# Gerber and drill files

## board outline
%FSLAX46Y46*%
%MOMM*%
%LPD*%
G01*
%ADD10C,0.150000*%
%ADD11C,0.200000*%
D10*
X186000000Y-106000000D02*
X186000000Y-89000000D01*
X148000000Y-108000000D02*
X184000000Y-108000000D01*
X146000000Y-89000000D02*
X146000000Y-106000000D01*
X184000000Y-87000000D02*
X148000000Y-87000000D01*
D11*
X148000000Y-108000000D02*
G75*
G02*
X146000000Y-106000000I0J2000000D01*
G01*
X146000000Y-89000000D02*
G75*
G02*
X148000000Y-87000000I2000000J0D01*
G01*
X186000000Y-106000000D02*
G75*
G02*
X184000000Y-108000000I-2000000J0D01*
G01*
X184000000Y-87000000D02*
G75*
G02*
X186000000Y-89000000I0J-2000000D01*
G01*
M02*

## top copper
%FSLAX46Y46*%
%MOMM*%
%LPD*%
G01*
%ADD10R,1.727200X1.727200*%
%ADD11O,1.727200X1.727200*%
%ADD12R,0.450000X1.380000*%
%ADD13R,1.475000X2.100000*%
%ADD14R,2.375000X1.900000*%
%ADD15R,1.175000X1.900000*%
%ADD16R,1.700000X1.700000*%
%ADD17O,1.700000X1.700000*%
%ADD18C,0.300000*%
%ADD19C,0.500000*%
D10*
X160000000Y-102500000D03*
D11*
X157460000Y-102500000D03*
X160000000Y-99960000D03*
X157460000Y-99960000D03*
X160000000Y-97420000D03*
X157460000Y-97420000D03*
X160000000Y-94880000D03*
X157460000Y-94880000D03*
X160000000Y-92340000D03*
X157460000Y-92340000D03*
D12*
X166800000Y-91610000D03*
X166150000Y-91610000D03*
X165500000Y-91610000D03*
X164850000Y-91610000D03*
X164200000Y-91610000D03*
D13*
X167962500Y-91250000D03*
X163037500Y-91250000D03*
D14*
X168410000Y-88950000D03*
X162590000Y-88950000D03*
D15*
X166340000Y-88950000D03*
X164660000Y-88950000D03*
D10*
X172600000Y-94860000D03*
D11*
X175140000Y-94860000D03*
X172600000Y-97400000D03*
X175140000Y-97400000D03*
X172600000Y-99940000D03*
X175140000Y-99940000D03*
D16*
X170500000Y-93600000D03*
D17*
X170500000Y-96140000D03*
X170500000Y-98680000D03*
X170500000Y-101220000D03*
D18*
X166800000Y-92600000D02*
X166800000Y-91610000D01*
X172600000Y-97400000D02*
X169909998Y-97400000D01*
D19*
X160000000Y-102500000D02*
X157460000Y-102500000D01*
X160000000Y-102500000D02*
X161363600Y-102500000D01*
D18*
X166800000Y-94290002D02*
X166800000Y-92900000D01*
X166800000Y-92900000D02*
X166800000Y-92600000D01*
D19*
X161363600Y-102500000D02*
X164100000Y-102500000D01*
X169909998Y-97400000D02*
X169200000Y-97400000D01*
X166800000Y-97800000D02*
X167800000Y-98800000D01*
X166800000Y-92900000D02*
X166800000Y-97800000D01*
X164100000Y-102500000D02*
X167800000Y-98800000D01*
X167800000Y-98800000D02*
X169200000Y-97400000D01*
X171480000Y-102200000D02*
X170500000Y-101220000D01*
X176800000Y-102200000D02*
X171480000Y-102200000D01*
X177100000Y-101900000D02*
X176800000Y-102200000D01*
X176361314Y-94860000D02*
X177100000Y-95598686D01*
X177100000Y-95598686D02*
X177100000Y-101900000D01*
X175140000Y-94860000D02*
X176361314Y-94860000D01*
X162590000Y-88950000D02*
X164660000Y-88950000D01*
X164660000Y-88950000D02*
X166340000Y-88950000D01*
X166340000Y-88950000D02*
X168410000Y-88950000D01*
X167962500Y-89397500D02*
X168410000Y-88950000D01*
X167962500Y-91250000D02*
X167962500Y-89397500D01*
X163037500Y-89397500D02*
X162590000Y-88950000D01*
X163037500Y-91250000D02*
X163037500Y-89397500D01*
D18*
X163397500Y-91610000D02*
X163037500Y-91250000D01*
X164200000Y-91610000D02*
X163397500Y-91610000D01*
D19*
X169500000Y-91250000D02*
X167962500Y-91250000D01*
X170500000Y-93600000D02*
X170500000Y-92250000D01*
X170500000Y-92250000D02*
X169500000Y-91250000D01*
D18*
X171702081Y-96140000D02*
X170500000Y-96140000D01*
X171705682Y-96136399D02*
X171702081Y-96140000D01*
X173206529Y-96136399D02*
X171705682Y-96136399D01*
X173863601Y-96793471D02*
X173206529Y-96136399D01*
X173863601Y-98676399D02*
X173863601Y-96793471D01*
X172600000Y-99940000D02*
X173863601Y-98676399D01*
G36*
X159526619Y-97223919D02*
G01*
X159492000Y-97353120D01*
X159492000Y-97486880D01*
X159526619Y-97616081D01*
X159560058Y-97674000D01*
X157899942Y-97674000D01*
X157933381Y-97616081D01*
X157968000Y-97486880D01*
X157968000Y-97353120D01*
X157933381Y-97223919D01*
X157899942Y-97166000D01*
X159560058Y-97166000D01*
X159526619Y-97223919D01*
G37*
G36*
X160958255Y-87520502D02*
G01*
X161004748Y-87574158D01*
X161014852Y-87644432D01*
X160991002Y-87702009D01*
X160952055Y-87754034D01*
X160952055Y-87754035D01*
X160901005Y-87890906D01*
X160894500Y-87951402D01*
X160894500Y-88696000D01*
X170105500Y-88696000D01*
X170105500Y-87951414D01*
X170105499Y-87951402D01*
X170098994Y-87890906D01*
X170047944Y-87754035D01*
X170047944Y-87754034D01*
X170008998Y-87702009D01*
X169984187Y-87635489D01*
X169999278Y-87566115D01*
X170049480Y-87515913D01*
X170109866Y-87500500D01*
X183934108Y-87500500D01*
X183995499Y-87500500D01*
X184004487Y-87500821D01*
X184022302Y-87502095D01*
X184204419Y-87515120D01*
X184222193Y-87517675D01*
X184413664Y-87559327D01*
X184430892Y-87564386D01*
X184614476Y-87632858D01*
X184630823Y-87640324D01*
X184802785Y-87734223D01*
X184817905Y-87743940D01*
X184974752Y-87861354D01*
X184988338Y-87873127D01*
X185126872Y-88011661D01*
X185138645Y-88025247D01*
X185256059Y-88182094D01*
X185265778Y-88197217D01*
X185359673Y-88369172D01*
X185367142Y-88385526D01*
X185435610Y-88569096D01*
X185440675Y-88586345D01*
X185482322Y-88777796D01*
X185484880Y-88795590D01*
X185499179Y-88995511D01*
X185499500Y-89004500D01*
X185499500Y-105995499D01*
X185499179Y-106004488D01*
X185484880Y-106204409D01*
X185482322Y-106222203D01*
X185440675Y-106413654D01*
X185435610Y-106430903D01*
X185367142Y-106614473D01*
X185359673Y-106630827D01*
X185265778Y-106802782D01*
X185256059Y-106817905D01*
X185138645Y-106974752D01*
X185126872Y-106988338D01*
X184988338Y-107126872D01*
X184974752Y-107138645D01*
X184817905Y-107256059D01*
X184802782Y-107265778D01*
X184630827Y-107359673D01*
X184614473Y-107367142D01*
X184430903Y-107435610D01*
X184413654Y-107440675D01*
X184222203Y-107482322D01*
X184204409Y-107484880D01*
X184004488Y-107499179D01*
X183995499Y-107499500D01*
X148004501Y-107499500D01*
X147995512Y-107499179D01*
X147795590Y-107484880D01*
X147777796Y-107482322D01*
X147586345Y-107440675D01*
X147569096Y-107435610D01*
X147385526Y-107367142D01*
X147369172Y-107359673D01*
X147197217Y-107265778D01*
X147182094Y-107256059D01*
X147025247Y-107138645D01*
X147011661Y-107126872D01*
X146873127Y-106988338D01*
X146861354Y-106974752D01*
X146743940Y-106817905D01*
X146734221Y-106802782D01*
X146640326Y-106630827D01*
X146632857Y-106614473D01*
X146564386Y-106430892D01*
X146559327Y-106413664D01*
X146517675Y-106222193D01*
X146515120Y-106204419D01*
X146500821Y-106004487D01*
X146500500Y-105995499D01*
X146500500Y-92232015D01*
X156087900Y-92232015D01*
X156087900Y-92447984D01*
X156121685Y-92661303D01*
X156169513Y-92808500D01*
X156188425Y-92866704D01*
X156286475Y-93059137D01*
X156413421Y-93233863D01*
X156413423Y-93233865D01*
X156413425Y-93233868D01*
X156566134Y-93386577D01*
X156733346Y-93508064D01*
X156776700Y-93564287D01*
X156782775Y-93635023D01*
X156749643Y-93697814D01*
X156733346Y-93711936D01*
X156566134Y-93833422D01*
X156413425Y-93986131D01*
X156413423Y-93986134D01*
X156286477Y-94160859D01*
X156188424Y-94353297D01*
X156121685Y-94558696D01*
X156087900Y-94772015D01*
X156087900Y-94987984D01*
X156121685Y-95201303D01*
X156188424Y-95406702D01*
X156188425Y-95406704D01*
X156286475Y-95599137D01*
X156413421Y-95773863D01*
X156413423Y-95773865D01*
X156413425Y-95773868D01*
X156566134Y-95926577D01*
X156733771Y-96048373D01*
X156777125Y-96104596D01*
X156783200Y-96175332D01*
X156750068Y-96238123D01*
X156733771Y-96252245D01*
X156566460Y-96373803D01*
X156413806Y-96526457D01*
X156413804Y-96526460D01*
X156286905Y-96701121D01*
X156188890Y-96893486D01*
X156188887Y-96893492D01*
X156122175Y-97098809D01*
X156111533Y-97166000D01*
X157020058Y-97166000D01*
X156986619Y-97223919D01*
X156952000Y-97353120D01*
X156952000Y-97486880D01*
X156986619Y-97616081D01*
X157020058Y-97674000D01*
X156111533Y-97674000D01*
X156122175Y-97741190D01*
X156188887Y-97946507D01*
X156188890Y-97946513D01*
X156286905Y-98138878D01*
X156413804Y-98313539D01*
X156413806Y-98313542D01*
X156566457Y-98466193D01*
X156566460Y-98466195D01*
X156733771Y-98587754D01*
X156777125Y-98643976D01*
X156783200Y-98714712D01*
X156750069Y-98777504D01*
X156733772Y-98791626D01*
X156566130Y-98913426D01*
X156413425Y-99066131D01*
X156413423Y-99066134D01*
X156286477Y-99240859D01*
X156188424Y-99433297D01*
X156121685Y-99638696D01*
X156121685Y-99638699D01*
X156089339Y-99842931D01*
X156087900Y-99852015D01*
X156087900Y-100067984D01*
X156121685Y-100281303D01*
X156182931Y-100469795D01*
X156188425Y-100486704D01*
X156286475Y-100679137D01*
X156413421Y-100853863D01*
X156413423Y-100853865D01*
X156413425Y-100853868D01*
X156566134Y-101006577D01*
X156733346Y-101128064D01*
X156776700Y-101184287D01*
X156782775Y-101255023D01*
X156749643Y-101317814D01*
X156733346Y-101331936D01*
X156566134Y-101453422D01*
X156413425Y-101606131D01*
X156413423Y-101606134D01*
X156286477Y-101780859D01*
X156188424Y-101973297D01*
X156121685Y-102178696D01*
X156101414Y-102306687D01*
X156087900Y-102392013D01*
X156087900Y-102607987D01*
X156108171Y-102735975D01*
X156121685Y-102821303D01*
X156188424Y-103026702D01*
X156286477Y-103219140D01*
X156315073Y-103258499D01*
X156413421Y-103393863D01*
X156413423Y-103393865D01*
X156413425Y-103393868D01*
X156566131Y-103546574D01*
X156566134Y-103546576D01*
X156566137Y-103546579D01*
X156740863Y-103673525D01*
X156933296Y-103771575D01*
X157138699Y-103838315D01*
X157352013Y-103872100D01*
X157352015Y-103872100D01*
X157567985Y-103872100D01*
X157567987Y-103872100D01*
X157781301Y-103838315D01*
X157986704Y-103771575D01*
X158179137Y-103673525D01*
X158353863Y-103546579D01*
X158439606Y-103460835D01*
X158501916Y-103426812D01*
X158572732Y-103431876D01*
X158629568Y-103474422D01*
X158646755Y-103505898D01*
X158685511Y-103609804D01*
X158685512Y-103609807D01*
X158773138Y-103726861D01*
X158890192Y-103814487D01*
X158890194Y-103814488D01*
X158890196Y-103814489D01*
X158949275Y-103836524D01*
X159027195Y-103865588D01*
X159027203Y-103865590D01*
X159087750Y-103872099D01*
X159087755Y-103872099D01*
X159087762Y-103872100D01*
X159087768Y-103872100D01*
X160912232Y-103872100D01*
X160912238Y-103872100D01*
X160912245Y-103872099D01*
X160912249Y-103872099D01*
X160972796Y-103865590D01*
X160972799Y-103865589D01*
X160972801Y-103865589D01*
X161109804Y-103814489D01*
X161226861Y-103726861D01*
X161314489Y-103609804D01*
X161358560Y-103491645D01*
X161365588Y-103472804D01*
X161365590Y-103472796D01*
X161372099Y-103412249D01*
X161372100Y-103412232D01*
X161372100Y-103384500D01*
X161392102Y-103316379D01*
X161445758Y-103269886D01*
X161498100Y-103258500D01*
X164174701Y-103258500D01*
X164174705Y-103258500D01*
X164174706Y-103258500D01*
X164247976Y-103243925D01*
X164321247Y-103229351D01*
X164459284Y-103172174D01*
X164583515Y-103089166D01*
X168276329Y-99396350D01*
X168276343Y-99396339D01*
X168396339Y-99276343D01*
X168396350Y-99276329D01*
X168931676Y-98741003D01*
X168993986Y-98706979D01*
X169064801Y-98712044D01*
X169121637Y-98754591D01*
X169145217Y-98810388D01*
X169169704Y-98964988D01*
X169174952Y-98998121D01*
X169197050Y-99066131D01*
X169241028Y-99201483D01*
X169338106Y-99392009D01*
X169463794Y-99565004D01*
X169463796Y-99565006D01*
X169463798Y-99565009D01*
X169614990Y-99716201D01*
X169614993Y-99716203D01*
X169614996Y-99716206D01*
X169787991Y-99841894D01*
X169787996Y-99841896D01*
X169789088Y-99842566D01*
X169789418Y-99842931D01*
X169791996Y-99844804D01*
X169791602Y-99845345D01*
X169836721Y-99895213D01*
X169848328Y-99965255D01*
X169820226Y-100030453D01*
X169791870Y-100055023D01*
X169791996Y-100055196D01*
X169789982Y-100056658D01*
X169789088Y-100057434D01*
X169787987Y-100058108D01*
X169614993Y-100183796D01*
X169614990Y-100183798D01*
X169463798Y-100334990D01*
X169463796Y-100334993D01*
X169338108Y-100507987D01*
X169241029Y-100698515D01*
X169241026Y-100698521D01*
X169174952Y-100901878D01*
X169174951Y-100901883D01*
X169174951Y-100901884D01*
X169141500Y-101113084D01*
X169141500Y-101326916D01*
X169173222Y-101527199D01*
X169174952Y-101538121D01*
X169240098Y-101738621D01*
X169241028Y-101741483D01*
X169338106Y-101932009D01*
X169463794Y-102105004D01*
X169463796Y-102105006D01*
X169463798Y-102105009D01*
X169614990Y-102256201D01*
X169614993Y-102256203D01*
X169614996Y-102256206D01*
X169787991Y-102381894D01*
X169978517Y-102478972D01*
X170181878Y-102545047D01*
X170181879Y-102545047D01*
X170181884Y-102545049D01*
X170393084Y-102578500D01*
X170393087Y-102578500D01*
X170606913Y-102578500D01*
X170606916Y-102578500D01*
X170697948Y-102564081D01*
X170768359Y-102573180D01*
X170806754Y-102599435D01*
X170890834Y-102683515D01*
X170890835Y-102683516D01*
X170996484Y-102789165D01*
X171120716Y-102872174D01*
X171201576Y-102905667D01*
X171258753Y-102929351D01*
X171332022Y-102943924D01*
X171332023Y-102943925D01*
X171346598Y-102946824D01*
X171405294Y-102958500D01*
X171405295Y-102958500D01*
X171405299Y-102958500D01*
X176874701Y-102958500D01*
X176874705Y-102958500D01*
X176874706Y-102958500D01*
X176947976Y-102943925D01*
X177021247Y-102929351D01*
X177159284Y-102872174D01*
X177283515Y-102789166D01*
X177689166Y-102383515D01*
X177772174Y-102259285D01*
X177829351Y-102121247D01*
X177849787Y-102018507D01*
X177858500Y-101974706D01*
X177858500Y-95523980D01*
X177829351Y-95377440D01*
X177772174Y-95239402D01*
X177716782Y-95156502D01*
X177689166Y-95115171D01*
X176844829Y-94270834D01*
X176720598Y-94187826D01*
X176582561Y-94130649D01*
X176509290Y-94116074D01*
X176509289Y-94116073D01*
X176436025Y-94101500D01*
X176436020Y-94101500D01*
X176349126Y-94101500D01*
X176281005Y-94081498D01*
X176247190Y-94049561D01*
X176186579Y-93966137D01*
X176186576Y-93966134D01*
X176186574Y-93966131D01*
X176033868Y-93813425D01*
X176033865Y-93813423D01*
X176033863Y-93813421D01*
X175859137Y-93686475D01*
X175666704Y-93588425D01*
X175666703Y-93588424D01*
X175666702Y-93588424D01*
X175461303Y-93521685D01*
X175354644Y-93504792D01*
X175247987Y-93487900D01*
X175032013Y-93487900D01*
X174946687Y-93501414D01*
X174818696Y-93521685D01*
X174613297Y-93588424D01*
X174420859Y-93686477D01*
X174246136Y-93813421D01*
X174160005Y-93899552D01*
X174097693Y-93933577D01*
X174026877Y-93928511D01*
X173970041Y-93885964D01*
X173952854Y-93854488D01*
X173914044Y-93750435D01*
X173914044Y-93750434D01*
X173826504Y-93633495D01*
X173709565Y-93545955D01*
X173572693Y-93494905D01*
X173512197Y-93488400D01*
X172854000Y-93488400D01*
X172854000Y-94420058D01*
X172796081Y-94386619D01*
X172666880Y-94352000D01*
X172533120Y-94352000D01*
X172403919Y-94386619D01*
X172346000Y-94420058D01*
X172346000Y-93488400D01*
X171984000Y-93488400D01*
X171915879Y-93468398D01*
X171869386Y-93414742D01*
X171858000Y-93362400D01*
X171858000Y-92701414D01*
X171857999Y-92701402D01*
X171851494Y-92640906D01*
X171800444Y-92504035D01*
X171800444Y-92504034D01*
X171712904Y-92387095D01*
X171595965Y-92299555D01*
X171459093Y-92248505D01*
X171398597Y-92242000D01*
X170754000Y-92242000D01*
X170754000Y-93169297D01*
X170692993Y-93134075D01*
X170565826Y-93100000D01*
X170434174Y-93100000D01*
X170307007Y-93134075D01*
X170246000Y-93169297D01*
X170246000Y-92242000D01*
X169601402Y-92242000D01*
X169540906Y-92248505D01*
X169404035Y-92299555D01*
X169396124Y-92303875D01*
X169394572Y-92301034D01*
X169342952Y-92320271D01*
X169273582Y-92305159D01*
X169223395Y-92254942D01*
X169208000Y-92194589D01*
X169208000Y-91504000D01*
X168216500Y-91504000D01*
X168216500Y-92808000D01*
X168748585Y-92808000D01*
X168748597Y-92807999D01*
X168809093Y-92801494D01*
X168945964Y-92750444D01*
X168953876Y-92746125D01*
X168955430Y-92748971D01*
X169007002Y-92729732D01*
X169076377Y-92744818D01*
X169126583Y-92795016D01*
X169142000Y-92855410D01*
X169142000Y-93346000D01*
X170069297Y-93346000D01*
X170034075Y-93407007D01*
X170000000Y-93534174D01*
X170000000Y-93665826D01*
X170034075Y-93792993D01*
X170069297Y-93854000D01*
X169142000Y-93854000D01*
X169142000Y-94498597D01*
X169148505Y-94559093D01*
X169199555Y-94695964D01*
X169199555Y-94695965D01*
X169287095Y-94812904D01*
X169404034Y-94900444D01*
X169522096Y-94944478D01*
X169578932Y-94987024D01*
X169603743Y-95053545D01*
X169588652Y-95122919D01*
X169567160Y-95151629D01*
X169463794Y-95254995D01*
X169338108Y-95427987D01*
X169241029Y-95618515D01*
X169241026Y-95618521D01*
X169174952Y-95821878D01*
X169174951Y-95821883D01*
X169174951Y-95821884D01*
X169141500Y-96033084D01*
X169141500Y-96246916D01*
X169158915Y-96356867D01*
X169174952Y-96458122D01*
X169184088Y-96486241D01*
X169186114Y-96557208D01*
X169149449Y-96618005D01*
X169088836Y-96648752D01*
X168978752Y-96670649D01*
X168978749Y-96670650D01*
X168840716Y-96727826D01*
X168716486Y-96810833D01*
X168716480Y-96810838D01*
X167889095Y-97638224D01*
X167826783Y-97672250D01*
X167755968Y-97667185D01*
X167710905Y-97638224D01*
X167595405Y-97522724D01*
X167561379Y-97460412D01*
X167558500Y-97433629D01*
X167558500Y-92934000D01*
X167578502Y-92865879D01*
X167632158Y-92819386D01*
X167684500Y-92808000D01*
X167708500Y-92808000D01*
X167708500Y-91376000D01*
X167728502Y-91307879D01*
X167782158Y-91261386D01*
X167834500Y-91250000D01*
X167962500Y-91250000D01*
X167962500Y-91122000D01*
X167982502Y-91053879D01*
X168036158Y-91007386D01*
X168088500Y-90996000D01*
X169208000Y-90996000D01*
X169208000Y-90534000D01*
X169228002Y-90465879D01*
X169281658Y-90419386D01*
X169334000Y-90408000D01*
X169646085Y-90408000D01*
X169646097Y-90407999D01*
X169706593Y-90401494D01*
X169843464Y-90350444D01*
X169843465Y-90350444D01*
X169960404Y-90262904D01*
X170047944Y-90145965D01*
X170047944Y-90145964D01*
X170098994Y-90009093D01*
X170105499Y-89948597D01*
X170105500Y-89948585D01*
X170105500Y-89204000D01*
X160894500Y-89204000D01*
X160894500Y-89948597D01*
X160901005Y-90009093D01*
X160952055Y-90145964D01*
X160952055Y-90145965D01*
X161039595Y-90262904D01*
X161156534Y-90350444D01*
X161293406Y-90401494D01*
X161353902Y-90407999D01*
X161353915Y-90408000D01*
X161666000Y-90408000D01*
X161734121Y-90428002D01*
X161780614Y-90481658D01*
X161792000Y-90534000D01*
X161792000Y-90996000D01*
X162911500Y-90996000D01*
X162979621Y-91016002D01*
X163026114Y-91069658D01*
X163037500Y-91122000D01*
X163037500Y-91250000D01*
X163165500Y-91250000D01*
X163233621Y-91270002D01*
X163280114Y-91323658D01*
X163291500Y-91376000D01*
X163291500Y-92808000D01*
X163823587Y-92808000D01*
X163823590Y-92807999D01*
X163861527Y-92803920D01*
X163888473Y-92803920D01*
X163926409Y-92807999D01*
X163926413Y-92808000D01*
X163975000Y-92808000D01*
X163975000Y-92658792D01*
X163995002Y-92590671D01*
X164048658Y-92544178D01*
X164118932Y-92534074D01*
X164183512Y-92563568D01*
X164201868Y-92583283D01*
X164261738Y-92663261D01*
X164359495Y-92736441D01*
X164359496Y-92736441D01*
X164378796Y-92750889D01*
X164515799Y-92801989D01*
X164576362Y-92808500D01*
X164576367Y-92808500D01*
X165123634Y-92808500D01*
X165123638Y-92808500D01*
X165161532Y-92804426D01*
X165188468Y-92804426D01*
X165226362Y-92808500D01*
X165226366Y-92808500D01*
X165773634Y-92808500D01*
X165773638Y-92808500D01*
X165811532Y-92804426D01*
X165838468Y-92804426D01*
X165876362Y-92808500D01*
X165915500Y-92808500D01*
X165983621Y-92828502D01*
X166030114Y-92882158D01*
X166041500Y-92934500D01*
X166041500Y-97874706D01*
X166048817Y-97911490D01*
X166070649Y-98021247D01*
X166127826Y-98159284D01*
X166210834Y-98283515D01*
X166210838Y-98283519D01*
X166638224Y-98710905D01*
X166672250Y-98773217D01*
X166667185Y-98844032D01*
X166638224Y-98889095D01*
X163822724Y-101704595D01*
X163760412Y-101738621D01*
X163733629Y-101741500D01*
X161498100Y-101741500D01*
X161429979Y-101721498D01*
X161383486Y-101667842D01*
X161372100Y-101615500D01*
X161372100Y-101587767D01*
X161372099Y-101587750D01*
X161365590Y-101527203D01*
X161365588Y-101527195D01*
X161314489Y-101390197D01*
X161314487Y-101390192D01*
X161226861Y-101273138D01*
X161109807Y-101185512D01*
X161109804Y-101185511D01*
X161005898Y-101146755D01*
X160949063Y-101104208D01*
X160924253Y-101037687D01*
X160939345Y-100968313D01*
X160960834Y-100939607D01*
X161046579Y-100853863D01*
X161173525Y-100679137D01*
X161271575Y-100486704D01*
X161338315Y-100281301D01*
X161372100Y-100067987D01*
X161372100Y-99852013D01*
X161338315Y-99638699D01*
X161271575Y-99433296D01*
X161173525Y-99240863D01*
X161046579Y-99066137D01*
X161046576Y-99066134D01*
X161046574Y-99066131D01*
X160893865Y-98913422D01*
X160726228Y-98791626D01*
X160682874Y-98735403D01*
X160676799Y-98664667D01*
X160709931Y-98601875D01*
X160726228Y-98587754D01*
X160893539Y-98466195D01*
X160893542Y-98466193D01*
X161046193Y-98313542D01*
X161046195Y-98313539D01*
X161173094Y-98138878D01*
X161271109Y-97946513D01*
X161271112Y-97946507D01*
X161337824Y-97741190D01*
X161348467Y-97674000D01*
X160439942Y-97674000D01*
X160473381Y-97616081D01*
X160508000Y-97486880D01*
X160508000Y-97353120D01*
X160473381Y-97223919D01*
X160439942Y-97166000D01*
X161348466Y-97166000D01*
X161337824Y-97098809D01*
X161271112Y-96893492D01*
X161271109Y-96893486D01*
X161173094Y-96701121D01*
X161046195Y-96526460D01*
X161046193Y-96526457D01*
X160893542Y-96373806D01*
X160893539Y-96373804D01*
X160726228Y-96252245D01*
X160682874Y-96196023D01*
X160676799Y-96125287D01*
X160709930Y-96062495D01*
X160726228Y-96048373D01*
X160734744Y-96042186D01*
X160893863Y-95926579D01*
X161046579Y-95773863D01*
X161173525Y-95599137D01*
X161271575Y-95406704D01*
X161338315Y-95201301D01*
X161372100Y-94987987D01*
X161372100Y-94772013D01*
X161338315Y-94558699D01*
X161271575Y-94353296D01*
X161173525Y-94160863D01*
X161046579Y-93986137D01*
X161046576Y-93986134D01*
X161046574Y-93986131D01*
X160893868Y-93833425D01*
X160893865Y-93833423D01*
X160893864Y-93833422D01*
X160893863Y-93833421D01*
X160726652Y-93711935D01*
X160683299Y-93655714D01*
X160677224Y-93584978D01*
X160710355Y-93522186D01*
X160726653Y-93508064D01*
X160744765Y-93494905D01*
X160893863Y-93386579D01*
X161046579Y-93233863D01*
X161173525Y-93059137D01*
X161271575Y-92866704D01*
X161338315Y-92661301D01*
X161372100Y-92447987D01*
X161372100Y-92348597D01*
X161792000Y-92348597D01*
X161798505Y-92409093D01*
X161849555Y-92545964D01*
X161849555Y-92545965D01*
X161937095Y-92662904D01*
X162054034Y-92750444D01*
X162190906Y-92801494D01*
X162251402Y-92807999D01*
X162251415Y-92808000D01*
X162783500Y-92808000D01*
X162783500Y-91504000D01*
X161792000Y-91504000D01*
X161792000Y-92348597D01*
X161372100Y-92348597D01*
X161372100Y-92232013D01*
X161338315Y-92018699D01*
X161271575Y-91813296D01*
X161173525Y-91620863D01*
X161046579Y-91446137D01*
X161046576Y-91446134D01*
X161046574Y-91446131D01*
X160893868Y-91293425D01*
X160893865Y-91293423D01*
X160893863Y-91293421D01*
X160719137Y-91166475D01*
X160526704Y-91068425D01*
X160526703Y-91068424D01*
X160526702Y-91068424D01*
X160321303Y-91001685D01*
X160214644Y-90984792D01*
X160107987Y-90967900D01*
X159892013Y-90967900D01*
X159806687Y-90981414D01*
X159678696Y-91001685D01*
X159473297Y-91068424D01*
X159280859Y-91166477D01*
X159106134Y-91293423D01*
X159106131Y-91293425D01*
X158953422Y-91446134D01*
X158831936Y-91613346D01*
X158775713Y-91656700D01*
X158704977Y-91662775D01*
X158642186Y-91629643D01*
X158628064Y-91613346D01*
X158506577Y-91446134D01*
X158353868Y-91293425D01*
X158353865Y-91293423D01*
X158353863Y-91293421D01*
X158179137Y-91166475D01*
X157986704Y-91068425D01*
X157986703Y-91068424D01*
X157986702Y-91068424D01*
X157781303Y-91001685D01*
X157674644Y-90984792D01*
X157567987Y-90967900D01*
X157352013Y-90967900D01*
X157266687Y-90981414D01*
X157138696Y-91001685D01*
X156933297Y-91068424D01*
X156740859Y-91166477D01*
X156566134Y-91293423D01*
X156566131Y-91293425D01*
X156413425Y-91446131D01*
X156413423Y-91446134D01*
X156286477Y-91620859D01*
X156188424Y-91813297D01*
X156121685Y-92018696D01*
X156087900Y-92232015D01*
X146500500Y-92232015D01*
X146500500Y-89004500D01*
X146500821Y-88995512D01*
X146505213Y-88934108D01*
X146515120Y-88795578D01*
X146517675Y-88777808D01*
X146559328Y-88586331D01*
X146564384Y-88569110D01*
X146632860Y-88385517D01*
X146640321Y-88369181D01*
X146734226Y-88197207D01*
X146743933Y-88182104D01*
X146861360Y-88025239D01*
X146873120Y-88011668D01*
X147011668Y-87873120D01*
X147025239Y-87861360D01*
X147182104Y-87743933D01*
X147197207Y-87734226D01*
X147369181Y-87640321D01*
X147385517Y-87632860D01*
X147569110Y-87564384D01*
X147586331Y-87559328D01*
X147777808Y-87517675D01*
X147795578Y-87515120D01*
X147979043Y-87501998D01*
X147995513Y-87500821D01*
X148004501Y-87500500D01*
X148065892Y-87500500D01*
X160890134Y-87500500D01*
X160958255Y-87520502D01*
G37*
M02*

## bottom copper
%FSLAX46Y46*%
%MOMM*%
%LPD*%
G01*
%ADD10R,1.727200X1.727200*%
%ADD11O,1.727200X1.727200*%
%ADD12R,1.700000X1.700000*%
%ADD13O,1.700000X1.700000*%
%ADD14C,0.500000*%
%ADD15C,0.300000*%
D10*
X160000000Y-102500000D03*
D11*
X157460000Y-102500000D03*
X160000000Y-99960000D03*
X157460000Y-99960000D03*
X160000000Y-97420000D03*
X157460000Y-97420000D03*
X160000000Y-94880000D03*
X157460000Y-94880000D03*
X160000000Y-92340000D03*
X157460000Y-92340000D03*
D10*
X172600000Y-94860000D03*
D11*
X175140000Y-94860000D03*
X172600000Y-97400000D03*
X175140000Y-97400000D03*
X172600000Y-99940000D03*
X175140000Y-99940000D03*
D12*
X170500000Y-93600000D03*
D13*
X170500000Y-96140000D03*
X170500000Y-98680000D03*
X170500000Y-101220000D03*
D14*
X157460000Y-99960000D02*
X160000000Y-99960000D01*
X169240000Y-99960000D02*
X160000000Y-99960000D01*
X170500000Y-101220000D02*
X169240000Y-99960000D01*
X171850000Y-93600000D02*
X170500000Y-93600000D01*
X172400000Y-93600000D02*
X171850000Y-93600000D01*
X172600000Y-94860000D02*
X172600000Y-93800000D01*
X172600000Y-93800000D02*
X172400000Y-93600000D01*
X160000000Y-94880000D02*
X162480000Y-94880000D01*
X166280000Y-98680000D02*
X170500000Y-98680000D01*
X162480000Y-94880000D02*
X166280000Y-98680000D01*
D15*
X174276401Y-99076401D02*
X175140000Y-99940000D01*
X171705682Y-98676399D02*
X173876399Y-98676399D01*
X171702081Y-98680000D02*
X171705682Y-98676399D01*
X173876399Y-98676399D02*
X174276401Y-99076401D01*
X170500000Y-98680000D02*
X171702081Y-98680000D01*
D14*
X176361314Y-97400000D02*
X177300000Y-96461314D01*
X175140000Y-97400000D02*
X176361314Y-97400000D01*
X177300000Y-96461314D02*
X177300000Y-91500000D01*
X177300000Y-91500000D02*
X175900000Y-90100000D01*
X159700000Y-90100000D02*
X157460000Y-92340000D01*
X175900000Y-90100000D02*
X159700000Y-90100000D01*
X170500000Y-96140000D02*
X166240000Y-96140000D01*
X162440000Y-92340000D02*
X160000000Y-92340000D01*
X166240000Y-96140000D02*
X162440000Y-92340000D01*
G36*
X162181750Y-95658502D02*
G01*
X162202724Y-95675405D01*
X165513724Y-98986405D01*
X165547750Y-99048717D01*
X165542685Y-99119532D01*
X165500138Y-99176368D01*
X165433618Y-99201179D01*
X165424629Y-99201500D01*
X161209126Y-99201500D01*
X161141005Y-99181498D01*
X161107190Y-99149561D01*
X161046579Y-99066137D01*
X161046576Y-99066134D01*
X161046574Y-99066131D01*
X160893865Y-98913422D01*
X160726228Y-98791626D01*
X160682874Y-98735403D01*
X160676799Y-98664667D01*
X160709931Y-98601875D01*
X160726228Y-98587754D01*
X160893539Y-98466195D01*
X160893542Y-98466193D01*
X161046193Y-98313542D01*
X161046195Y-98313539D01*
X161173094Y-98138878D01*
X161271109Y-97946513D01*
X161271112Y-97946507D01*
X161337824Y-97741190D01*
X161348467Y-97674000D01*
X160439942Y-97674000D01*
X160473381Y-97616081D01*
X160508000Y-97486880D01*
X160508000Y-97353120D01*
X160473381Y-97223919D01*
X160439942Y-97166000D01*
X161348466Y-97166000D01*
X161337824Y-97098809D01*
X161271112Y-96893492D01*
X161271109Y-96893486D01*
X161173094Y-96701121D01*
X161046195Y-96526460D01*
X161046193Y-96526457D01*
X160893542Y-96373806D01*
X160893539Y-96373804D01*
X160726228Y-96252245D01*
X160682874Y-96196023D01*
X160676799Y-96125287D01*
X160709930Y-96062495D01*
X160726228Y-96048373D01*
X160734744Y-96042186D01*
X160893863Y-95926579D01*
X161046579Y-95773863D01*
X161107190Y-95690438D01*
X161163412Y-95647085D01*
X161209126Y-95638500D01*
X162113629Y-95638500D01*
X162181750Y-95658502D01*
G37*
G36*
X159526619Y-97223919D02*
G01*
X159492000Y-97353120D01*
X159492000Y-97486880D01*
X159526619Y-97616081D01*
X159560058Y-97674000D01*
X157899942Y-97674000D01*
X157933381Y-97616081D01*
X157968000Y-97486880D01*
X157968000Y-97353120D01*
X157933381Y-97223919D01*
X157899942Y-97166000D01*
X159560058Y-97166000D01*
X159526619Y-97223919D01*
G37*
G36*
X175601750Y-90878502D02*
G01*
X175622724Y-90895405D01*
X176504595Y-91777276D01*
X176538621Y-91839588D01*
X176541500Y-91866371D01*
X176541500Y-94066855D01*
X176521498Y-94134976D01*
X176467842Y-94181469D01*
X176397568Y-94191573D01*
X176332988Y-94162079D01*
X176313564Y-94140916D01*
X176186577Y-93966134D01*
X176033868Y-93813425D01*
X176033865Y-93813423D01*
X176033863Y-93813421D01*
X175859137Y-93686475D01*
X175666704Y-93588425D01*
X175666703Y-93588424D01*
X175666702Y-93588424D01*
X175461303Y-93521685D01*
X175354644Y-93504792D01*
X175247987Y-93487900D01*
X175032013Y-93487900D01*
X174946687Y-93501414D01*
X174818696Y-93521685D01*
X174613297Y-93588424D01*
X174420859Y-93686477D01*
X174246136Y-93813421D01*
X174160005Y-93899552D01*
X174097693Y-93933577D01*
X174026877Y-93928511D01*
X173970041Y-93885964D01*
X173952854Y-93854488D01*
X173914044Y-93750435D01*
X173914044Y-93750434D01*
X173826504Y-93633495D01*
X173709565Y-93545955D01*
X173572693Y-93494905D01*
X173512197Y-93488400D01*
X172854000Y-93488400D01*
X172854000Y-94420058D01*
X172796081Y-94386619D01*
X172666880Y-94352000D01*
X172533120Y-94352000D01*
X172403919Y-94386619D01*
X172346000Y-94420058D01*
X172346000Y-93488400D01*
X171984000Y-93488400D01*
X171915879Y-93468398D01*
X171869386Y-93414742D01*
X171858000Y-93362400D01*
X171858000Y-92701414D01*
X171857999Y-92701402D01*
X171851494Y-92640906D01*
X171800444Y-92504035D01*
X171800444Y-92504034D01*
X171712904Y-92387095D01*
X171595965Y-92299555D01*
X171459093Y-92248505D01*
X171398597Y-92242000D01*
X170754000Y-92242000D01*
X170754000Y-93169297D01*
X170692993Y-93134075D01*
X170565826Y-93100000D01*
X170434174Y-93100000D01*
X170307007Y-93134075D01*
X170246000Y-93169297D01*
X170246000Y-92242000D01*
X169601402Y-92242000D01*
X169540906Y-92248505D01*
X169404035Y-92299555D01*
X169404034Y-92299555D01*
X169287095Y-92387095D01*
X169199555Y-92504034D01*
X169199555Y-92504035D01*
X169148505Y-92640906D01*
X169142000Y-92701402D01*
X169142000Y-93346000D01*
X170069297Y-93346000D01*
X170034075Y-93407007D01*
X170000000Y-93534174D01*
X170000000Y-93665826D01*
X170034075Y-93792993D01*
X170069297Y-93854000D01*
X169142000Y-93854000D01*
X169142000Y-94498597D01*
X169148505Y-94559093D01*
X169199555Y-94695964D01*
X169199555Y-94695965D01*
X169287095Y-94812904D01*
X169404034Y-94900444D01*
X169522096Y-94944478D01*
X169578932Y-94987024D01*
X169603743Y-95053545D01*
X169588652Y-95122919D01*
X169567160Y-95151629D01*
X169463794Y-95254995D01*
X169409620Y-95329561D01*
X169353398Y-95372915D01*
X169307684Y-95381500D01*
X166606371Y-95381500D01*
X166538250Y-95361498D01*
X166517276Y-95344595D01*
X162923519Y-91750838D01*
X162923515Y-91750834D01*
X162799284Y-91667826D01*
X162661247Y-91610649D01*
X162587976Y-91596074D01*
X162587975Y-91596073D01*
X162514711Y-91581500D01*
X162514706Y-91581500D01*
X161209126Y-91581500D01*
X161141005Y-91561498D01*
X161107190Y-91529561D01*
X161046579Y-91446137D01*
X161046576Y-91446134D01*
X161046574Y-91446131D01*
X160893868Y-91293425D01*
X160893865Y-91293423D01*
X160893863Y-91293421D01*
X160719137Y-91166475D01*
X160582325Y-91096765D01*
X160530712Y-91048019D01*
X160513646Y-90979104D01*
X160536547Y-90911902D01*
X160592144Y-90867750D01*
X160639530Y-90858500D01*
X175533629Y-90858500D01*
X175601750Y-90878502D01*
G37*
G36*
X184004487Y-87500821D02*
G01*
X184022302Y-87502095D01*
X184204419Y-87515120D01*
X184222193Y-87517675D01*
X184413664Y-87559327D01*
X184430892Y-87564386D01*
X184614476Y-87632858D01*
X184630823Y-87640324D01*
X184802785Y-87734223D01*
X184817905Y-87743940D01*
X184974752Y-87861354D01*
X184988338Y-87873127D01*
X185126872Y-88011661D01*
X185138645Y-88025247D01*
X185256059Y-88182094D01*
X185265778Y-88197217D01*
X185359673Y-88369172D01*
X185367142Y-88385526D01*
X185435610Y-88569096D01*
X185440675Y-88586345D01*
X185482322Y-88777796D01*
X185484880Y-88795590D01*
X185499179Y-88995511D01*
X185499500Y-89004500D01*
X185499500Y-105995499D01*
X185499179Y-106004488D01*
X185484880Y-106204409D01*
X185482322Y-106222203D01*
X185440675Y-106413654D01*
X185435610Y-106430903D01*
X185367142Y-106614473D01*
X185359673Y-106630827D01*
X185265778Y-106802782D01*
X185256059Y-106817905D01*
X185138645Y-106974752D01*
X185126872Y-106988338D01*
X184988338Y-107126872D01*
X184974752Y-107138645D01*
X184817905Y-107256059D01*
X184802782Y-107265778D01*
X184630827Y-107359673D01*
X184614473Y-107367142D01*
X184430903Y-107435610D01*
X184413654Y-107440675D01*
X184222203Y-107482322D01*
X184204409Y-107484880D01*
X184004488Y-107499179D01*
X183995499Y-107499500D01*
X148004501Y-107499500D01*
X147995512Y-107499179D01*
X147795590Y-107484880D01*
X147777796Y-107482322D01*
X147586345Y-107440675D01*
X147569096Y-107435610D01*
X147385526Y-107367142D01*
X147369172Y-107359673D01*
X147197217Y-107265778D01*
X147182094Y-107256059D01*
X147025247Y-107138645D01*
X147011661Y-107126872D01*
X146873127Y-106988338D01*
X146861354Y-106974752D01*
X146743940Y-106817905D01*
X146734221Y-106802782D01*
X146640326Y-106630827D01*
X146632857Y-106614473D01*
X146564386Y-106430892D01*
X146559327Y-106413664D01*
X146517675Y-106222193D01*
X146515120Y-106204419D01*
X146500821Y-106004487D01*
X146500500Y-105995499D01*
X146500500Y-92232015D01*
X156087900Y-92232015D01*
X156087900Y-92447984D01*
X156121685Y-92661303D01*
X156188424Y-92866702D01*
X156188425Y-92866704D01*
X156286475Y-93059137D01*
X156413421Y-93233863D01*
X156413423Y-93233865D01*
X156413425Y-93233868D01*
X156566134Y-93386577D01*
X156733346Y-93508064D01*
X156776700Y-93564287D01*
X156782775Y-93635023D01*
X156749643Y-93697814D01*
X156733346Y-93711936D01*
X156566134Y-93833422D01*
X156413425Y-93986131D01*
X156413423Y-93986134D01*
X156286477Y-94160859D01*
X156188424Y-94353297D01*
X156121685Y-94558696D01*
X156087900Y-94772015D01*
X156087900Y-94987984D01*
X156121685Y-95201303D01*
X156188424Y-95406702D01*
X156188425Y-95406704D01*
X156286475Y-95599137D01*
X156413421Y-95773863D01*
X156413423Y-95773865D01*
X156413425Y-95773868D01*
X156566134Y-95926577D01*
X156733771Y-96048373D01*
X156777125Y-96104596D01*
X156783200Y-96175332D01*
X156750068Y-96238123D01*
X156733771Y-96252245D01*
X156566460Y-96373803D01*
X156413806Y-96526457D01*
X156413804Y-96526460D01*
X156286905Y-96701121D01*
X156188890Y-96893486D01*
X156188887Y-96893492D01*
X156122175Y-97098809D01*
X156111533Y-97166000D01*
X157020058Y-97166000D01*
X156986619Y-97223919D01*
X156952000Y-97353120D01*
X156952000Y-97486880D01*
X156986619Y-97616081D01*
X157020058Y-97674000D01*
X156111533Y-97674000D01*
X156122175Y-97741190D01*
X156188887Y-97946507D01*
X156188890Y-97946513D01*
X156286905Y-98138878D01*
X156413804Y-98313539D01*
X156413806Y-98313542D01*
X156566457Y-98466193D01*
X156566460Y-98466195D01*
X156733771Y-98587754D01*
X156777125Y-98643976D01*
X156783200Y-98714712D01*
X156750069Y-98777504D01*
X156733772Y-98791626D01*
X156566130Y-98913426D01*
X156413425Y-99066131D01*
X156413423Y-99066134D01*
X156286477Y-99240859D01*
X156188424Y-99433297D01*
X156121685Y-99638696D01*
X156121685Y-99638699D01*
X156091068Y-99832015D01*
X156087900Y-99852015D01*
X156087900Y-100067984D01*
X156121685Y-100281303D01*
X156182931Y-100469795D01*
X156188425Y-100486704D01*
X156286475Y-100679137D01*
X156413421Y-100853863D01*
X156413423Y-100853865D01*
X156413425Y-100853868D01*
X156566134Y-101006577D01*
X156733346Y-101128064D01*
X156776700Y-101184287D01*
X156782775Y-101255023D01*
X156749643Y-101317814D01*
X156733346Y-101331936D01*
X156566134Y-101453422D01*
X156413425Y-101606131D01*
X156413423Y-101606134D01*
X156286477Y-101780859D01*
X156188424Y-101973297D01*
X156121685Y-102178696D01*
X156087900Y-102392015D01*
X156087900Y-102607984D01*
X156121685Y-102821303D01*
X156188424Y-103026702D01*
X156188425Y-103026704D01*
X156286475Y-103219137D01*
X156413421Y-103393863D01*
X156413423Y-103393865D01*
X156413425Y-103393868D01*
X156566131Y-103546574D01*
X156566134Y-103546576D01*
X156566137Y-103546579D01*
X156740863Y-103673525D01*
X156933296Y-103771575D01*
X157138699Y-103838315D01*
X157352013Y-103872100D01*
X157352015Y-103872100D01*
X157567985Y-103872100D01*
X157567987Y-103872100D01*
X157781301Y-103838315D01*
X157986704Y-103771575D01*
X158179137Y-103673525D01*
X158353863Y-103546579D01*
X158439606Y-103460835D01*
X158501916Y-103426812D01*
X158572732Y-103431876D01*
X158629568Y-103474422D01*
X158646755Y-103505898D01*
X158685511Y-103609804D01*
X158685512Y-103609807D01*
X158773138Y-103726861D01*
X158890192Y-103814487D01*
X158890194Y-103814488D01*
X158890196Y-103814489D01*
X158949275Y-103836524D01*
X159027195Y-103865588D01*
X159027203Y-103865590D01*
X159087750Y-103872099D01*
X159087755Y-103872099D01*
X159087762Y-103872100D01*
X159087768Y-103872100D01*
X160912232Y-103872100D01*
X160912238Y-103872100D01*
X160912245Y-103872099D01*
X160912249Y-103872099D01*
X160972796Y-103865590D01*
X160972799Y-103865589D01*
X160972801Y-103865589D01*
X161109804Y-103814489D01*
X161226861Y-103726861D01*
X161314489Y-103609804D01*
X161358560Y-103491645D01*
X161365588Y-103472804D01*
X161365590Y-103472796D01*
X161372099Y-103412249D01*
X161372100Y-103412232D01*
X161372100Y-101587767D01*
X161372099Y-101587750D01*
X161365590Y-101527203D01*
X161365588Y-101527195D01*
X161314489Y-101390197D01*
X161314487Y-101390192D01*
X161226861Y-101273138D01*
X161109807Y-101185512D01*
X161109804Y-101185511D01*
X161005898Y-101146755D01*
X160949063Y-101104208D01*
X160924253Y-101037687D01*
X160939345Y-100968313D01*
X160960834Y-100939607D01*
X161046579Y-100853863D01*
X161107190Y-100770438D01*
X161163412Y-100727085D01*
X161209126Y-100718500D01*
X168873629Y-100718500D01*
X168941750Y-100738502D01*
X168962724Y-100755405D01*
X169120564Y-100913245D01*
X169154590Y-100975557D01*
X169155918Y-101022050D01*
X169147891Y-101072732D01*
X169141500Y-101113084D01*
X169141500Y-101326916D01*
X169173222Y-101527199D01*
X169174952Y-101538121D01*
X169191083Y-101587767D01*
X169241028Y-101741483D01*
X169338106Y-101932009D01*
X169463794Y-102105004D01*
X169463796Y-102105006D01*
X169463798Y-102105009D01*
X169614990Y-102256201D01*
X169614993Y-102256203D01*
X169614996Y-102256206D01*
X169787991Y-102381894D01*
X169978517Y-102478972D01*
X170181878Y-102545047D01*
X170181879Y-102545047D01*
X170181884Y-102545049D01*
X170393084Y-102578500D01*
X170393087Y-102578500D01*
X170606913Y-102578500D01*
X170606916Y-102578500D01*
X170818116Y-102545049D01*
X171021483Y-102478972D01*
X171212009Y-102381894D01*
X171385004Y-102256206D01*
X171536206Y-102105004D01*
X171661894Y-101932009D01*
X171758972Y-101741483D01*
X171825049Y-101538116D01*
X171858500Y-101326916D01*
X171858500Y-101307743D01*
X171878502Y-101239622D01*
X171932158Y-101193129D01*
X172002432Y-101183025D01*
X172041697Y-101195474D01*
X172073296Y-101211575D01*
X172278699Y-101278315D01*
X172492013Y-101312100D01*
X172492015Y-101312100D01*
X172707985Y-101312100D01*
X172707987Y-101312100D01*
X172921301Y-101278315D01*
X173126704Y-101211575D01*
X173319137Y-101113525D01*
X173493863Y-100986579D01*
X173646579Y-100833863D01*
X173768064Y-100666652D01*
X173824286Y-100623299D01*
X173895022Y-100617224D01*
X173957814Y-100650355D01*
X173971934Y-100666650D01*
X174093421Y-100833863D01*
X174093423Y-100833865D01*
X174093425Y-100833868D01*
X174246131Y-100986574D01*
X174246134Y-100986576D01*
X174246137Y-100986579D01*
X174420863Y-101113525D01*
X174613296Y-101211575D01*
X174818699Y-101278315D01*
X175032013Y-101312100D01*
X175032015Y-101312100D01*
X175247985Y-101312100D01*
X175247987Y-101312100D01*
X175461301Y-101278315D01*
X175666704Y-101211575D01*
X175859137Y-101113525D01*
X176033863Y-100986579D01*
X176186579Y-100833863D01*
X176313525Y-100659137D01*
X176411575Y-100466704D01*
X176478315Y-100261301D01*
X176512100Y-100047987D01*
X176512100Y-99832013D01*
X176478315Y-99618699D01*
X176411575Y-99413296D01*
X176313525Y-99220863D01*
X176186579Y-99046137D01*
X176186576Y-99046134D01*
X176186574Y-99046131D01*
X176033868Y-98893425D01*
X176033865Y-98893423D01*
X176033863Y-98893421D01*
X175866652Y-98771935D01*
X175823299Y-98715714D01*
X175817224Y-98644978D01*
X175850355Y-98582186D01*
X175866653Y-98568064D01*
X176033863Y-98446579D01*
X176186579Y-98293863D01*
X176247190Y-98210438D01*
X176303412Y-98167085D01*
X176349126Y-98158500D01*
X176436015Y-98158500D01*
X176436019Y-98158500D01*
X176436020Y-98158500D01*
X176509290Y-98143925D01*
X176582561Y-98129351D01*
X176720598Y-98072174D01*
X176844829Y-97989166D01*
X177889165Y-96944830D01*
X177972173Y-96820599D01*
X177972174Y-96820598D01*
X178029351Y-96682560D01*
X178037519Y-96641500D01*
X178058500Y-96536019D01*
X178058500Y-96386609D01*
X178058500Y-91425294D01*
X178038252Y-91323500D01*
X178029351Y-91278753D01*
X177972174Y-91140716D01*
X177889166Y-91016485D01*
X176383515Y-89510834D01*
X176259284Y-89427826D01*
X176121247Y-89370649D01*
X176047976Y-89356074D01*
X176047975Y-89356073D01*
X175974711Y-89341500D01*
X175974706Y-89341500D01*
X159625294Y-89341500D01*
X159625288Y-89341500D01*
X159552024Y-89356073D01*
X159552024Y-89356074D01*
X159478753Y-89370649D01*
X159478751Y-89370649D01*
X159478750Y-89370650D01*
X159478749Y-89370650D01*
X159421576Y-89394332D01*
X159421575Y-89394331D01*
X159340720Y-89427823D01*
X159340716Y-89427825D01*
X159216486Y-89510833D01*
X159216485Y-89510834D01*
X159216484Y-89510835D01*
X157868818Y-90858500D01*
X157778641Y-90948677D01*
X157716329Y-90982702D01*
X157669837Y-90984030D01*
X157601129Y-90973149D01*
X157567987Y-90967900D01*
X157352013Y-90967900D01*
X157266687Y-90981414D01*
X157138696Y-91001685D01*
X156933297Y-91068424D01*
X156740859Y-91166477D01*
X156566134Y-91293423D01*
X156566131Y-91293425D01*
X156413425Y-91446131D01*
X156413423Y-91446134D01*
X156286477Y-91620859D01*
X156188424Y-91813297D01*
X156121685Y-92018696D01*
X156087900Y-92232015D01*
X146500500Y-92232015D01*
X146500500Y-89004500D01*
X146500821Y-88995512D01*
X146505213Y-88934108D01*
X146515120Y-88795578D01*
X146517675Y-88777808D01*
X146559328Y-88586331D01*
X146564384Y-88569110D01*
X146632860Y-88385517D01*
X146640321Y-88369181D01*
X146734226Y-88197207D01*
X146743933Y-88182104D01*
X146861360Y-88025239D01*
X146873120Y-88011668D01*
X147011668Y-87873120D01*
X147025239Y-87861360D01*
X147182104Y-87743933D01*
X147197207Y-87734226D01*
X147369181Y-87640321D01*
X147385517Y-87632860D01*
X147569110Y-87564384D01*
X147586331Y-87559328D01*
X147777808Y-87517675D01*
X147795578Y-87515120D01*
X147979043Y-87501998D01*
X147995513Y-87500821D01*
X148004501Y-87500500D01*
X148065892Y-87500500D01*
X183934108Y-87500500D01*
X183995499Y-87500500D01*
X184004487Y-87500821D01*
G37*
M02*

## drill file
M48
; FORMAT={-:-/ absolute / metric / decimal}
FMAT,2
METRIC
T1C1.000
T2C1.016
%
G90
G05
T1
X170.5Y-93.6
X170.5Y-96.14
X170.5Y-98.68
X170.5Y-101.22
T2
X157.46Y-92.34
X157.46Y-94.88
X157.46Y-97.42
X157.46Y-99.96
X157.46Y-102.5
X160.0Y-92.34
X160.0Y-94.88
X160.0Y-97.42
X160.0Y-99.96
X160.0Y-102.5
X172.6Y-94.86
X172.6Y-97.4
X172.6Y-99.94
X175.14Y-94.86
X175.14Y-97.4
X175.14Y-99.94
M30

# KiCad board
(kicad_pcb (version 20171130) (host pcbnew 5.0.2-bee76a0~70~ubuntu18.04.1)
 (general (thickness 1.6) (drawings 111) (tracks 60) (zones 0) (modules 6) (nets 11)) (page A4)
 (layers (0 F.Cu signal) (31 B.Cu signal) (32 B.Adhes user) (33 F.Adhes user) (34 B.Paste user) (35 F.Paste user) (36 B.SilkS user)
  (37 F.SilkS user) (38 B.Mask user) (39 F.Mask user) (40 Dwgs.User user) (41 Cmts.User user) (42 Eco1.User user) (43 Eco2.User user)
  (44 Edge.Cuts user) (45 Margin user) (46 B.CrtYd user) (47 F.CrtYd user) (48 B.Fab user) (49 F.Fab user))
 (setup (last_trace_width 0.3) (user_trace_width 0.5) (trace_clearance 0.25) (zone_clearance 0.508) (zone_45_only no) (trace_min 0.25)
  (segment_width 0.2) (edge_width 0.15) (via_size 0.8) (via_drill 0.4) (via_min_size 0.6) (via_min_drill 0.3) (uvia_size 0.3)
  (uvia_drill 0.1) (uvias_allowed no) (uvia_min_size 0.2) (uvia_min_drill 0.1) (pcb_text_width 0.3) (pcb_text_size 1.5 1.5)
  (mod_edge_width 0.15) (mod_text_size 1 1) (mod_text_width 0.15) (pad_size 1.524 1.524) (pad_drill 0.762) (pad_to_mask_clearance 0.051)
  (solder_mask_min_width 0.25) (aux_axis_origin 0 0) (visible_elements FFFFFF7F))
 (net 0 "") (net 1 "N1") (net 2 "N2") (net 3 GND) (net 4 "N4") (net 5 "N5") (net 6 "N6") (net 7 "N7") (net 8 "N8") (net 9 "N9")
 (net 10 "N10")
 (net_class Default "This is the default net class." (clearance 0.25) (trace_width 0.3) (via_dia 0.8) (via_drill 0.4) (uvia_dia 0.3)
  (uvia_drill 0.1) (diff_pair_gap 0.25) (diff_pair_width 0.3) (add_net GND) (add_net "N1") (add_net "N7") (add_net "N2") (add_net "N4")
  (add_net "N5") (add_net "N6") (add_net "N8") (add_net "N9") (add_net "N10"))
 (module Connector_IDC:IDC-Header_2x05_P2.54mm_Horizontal (layer F.Cu) (at 160 102.5 180)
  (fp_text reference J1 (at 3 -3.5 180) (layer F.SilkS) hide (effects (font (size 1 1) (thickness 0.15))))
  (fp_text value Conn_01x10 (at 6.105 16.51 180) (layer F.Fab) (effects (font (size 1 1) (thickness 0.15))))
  (pad 1 thru_hole rect (at 0 0 180) (size 1.7272 1.7272) (drill 1.016) (layers *.Cu *.Mask) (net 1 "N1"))
  (pad 2 thru_hole oval (at 2.54 0 180) (size 1.7272 1.7272) (drill 1.016) (layers *.Cu *.Mask) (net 1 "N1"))
  (pad 3 thru_hole oval (at 0 2.54 180) (size 1.7272 1.7272) (drill 1.016) (layers *.Cu *.Mask) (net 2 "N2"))
  (pad 4 thru_hole oval (at 2.54 2.54 180) (size 1.7272 1.7272) (drill 1.016) (layers *.Cu *.Mask) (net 2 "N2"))
  (pad 5 thru_hole oval (at 0 5.08 180) (size 1.7272 1.7272) (drill 1.016) (layers *.Cu *.Mask) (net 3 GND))
  (pad 6 thru_hole oval (at 2.54 5.08 180) (size 1.7272 1.7272) (drill 1.016) (layers *.Cu *.Mask) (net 3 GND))
  (pad 7 thru_hole oval (at 0 7.62 180) (size 1.7272 1.7272) (drill 1.016) (layers *.Cu *.Mask) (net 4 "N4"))
  (pad 8 thru_hole oval (at 2.54 7.62 180) (size 1.7272 1.7272) (drill 1.016) (layers *.Cu *.Mask) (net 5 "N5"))
  (pad 9 thru_hole oval (at 0 10.16 180) (size 1.7272 1.7272) (drill 1.016) (layers *.Cu *.Mask) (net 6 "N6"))
  (pad 10 thru_hole oval (at 2.54 10.16 180) (size 1.7272 1.7272) (drill 1.016) (layers *.Cu *.Mask) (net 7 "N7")))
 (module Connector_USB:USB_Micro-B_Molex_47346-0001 (layer F.Cu) (at 165.5 90.15 180)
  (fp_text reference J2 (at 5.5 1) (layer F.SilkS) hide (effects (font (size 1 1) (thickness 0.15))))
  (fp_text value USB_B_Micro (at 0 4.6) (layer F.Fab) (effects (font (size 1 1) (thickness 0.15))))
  (pad 1 smd rect (at -1.3 -1.46 180) (size 0.45 1.38) (layers F.Cu F.Paste F.Mask) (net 1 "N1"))
  (pad 2 smd rect (at -0.65 -1.46 180) (size 0.45 1.38) (layers F.Cu F.Paste F.Mask) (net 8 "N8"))
  (pad 3 smd rect (at 0 -1.46 180) (size 0.45 1.38) (layers F.Cu F.Paste F.Mask) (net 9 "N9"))
  (pad 4 smd rect (at 0.65 -1.46 180) (size 0.45 1.38) (layers F.Cu F.Paste F.Mask) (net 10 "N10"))
  (pad 5 smd rect (at 1.3 -1.46 180) (size 0.45 1.38) (layers F.Cu F.Paste F.Mask) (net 3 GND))
  (pad 6 smd rect (at -2.4625 -1.1 180) (size 1.475 2.1) (layers F.Cu F.Paste F.Mask) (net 3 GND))
  (pad 6 smd rect (at 2.4625 -1.1 180) (size 1.475 2.1) (layers F.Cu F.Paste F.Mask) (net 3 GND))
  (pad 6 smd rect (at -2.91 1.2 180) (size 2.375 1.9) (layers F.Cu F.Paste F.Mask) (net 3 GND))
  (pad 6 smd rect (at 2.91 1.2 180) (size 2.375 1.9) (layers F.Cu F.Paste F.Mask) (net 3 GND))
  (pad 6 smd rect (at -0.84 1.2 180) (size 1.175 1.9) (layers F.Cu F.Paste F.Mask) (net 3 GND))
  (pad 6 smd rect (at 0.84 1.2 180) (size 1.175 1.9) (layers F.Cu F.Paste F.Mask) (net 3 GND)))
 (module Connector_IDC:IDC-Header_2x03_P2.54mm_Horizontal (layer F.Cu) (at 172.6 94.86)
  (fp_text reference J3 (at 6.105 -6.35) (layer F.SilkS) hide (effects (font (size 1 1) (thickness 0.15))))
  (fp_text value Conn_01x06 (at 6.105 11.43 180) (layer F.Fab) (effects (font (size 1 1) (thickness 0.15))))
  (pad 1 thru_hole rect (at 0 0) (size 1.7272 1.7272) (drill 1.016) (layers *.Cu *.Mask) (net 3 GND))
  (pad 2 thru_hole oval (at 2.54 0) (size 1.7272 1.7272) (drill 1.016) (layers *.Cu *.Mask) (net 2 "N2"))
  (pad 3 thru_hole oval (at 0 2.54) (size 1.7272 1.7272) (drill 1.016) (layers *.Cu *.Mask) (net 1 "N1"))
  (pad 4 thru_hole oval (at 2.54 2.54) (size 1.7272 1.7272) (drill 1.016) (layers *.Cu *.Mask) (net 7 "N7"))
  (pad 5 thru_hole oval (at 0 5.08) (size 1.7272 1.7272) (drill 1.016) (layers *.Cu *.Mask) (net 6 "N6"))
  (pad 6 thru_hole oval (at 2.54 5.08) (size 1.7272 1.7272) (drill 1.016) (layers *.Cu *.Mask) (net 4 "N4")))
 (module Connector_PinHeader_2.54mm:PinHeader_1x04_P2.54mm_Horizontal (layer F.Cu) (at 170.5 93.6)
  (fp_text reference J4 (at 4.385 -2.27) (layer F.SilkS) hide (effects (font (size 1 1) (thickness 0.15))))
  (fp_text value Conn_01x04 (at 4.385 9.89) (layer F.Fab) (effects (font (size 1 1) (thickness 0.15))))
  (pad 1 thru_hole rect (at 0 0) (size 1.7 1.7) (drill 1) (layers *.Cu *.Mask) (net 3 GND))
  (pad 2 thru_hole oval (at 0 2.54) (size 1.7 1.7) (drill 1) (layers *.Cu *.Mask) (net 6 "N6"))
  (pad 3 thru_hole oval (at 0 5.08) (size 1.7 1.7) (drill 1) (layers *.Cu *.Mask) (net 4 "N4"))
  (pad 4 thru_hole oval (at 0 7.62) (size 1.7 1.7) (drill 1) (layers *.Cu *.Mask) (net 2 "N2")))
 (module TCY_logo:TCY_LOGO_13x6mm (layer B.Cu) (at 165.25 97.55 270)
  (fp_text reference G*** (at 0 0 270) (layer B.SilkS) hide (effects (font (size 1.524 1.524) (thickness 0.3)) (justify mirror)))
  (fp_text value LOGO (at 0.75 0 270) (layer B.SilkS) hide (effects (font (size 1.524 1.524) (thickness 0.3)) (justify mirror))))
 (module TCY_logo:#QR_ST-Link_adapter (layer B.Cu) (at 180.9 97.45)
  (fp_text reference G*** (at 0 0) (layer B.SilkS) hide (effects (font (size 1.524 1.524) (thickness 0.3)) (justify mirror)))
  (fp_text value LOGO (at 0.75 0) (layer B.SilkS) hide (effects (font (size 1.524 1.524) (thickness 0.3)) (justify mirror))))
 (gr_line (start 186 106) (end 186 89) (layer Edge.Cuts) (width 0.15))
 (gr_line (start 148 108) (end 184 108) (layer Edge.Cuts) (width 0.15))
 (gr_line (start 146 89) (end 146 106) (layer Edge.Cuts) (width 0.15))
 (gr_line (start 184 87) (end 148 87) (layer Edge.Cuts) (width 0.15))
 (gr_arc (start 148 106) (end 146 106) (angle -90) (layer Edge.Cuts) (width 0.2))
 (gr_arc (start 148 89) (end 148 87) (angle -90) (layer Edge.Cuts) (width 0.2))
 (gr_arc (start 184 106) (end 184 108) (angle -90) (layer Edge.Cuts) (width 0.2))
 (gr_arc (start 184 89) (end 186 89) (angle -90) (layer Edge.Cuts) (width 0.2))
 (segment (start 166.8 92.6) (end 166.8 91.61) (width 0.3) (layer F.Cu) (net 1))
 (segment (start 172.6 97.4) (end 169.909998 97.4) (width 0.3) (layer F.Cu) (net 1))
 (segment (start 160 102.5) (end 157.46 102.5) (width 0.5) (layer F.Cu) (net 1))
 (segment (start 160 102.5) (end 161.3636 102.5) (width 0.5) (layer F.Cu) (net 1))
 (segment (start 166.8 94.290002) (end 166.8 92.9) (width 0.3) (layer F.Cu) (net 1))
 (segment (start 166.8 92.9) (end 166.8 92.6) (width 0.3) (layer F.Cu) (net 1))
 (segment (start 161.3636 102.5) (end 164.1 102.5) (width 0.5) (layer F.Cu) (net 1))
 (segment (start 169.909998 97.4) (end 169.2 97.4) (width 0.5) (layer F.Cu) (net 1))
 (segment (start 166.8 97.8) (end 167.8 98.8) (width 0.5) (layer F.Cu) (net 1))
 (segment (start 166.8 92.9) (end 166.8 97.8) (width 0.5) (layer F.Cu) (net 1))
 (segment (start 164.1 102.5) (end 167.8 98.8) (width 0.5) (layer F.Cu) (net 1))
 (segment (start 167.8 98.8) (end 169.2 97.4) (width 0.5) (layer F.Cu) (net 1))
 (segment (start 171.48 102.2) (end 170.5 101.22) (width 0.5) (layer F.Cu) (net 2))
 (segment (start 176.8 102.2) (end 171.48 102.2) (width 0.5) (layer F.Cu) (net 2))
 (segment (start 177.1 101.9) (end 176.8 102.2) (width 0.5) (layer F.Cu) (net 2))
 (segment (start 176.361314 94.86) (end 177.1 95.598686) (width 0.5) (layer F.Cu) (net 2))
 (segment (start 177.1 95.598686) (end 177.1 101.9) (width 0.5) (layer F.Cu) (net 2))
 (segment (start 175.14 94.86) (end 176.361314 94.86) (width 0.5) (layer F.Cu) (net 2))
 (segment (start 157.46 99.96) (end 160 99.96) (width 0.5) (layer B.Cu) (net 2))
 (segment (start 169.24 99.96) (end 160 99.96) (width 0.5) (layer B.Cu) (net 2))
 (segment (start 170.5 101.22) (end 169.24 99.96) (width 0.5) (layer B.Cu) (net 2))
 (segment (start 162.59 88.95) (end 164.66 88.95) (width 0.5) (layer F.Cu) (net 3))
 (segment (start 164.66 88.95) (end 166.34 88.95) (width 0.5) (layer F.Cu) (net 3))
 (segment (start 166.34 88.95) (end 168.41 88.95) (width 0.5) (layer F.Cu) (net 3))
 (segment (start 167.9625 89.3975) (end 168.41 88.95) (width 0.5) (layer F.Cu) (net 3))
 (segment (start 167.9625 91.25) (end 167.9625 89.3975) (width 0.5) (layer F.Cu) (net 3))
 (segment (start 163.0375 89.3975) (end 162.59 88.95) (width 0.5) (layer F.Cu) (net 3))
 (segment (start 163.0375 91.25) (end 163.0375 89.3975) (width 0.5) (layer F.Cu) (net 3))
 (segment (start 163.3975 91.61) (end 163.0375 91.25) (width 0.3) (layer F.Cu) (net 3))
 (segment (start 164.2 91.61) (end 163.3975 91.61) (width 0.3) (layer F.Cu) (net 3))
 (segment (start 171.85 93.6) (end 170.5 93.6) (width 0.5) (layer B.Cu) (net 3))
 (segment (start 172.4 93.6) (end 171.85 93.6) (width 0.5) (layer B.Cu) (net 3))
 (segment (start 172.6 94.86) (end 172.6 93.8) (width 0.5) (layer B.Cu) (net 3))
 (segment (start 172.6 93.8) (end 172.4 93.6) (width 0.5) (layer B.Cu) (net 3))
 (segment (start 169.5 91.25) (end 167.9625 91.25) (width 0.5) (layer F.Cu) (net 3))
 (segment (start 170.5 93.6) (end 170.5 92.25) (width 0.5) (layer F.Cu) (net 3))
 (segment (start 170.5 92.25) (end 169.5 91.25) (width 0.5) (layer F.Cu) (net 3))
 (segment (start 160 94.88) (end 162.48 94.88) (width 0.5) (layer B.Cu) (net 4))
 (segment (start 166.28 98.68) (end 170.5 98.68) (width 0.5) (layer B.Cu) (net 4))
 (segment (start 162.48 94.88) (end 166.28 98.68) (width 0.5) (layer B.Cu) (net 4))
 (segment (start 174.276401 99.076401) (end 175.14 99.94) (width 0.3) (layer B.Cu) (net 4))
 (segment (start 171.705682 98.676399) (end 173.876399 98.676399) (width 0.3) (layer B.Cu) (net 4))
 (segment (start 171.702081 98.68) (end 171.705682 98.676399) (width 0.3) (layer B.Cu) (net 4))
 (segment (start 173.876399 98.676399) (end 174.276401 99.076401) (width 0.3) (layer B.Cu) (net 4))
 (segment (start 170.5 98.68) (end 171.702081 98.68) (width 0.3) (layer B.Cu) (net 4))
 (segment (start 176.361314 97.4) (end 177.3 96.461314) (width 0.5) (layer B.Cu) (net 7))
 (segment (start 175.14 97.4) (end 176.361314 97.4) (width 0.5) (layer B.Cu) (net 7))
 (segment (start 177.3 96.461314) (end 177.3 91.5) (width 0.5) (layer B.Cu) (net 7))
 (segment (start 177.3 91.5) (end 175.9 90.1) (width 0.5) (layer B.Cu) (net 7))
 (segment (start 159.7 90.1) (end 157.46 92.34) (width 0.5) (layer B.Cu) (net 7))
 (segment (start 175.9 90.1) (end 159.7 90.1) (width 0.5) (layer B.Cu) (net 7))
 (segment (start 171.702081 96.14) (end 170.5 96.14) (width 0.3) (layer F.Cu) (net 6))
 (segment (start 171.705682 96.136399) (end 171.702081 96.14) (width 0.3) (layer F.Cu) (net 6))
 (segment (start 173.206529 96.136399) (end 171.705682 96.136399) (width 0.3) (layer F.Cu) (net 6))
 (segment (start 173.863601 96.793471) (end 173.206529 96.136399) (width 0.3) (layer F.Cu) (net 6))
 (segment (start 173.863601 98.676399) (end 173.863601 96.793471) (width 0.3) (layer F.Cu) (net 6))
 (segment (start 172.6 99.94) (end 173.863601 98.676399) (width 0.3) (layer F.Cu) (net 6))
 (segment (start 170.5 96.14) (end 166.24 96.14) (width 0.5) (layer B.Cu) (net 6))
 (segment (start 162.44 92.34) (end 160 92.34) (width 0.5) (layer B.Cu) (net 6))
 (segment (start 166.24 96.14) (end 162.44 92.34) (width 0.5) (layer B.Cu) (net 6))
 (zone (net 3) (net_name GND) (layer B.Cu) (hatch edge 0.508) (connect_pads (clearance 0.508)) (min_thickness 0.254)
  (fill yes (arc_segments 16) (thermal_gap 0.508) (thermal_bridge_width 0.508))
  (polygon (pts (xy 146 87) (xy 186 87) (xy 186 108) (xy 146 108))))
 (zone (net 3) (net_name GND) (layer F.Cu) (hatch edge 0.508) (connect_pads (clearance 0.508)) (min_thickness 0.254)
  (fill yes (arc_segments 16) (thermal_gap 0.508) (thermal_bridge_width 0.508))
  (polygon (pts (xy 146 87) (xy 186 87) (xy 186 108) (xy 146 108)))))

